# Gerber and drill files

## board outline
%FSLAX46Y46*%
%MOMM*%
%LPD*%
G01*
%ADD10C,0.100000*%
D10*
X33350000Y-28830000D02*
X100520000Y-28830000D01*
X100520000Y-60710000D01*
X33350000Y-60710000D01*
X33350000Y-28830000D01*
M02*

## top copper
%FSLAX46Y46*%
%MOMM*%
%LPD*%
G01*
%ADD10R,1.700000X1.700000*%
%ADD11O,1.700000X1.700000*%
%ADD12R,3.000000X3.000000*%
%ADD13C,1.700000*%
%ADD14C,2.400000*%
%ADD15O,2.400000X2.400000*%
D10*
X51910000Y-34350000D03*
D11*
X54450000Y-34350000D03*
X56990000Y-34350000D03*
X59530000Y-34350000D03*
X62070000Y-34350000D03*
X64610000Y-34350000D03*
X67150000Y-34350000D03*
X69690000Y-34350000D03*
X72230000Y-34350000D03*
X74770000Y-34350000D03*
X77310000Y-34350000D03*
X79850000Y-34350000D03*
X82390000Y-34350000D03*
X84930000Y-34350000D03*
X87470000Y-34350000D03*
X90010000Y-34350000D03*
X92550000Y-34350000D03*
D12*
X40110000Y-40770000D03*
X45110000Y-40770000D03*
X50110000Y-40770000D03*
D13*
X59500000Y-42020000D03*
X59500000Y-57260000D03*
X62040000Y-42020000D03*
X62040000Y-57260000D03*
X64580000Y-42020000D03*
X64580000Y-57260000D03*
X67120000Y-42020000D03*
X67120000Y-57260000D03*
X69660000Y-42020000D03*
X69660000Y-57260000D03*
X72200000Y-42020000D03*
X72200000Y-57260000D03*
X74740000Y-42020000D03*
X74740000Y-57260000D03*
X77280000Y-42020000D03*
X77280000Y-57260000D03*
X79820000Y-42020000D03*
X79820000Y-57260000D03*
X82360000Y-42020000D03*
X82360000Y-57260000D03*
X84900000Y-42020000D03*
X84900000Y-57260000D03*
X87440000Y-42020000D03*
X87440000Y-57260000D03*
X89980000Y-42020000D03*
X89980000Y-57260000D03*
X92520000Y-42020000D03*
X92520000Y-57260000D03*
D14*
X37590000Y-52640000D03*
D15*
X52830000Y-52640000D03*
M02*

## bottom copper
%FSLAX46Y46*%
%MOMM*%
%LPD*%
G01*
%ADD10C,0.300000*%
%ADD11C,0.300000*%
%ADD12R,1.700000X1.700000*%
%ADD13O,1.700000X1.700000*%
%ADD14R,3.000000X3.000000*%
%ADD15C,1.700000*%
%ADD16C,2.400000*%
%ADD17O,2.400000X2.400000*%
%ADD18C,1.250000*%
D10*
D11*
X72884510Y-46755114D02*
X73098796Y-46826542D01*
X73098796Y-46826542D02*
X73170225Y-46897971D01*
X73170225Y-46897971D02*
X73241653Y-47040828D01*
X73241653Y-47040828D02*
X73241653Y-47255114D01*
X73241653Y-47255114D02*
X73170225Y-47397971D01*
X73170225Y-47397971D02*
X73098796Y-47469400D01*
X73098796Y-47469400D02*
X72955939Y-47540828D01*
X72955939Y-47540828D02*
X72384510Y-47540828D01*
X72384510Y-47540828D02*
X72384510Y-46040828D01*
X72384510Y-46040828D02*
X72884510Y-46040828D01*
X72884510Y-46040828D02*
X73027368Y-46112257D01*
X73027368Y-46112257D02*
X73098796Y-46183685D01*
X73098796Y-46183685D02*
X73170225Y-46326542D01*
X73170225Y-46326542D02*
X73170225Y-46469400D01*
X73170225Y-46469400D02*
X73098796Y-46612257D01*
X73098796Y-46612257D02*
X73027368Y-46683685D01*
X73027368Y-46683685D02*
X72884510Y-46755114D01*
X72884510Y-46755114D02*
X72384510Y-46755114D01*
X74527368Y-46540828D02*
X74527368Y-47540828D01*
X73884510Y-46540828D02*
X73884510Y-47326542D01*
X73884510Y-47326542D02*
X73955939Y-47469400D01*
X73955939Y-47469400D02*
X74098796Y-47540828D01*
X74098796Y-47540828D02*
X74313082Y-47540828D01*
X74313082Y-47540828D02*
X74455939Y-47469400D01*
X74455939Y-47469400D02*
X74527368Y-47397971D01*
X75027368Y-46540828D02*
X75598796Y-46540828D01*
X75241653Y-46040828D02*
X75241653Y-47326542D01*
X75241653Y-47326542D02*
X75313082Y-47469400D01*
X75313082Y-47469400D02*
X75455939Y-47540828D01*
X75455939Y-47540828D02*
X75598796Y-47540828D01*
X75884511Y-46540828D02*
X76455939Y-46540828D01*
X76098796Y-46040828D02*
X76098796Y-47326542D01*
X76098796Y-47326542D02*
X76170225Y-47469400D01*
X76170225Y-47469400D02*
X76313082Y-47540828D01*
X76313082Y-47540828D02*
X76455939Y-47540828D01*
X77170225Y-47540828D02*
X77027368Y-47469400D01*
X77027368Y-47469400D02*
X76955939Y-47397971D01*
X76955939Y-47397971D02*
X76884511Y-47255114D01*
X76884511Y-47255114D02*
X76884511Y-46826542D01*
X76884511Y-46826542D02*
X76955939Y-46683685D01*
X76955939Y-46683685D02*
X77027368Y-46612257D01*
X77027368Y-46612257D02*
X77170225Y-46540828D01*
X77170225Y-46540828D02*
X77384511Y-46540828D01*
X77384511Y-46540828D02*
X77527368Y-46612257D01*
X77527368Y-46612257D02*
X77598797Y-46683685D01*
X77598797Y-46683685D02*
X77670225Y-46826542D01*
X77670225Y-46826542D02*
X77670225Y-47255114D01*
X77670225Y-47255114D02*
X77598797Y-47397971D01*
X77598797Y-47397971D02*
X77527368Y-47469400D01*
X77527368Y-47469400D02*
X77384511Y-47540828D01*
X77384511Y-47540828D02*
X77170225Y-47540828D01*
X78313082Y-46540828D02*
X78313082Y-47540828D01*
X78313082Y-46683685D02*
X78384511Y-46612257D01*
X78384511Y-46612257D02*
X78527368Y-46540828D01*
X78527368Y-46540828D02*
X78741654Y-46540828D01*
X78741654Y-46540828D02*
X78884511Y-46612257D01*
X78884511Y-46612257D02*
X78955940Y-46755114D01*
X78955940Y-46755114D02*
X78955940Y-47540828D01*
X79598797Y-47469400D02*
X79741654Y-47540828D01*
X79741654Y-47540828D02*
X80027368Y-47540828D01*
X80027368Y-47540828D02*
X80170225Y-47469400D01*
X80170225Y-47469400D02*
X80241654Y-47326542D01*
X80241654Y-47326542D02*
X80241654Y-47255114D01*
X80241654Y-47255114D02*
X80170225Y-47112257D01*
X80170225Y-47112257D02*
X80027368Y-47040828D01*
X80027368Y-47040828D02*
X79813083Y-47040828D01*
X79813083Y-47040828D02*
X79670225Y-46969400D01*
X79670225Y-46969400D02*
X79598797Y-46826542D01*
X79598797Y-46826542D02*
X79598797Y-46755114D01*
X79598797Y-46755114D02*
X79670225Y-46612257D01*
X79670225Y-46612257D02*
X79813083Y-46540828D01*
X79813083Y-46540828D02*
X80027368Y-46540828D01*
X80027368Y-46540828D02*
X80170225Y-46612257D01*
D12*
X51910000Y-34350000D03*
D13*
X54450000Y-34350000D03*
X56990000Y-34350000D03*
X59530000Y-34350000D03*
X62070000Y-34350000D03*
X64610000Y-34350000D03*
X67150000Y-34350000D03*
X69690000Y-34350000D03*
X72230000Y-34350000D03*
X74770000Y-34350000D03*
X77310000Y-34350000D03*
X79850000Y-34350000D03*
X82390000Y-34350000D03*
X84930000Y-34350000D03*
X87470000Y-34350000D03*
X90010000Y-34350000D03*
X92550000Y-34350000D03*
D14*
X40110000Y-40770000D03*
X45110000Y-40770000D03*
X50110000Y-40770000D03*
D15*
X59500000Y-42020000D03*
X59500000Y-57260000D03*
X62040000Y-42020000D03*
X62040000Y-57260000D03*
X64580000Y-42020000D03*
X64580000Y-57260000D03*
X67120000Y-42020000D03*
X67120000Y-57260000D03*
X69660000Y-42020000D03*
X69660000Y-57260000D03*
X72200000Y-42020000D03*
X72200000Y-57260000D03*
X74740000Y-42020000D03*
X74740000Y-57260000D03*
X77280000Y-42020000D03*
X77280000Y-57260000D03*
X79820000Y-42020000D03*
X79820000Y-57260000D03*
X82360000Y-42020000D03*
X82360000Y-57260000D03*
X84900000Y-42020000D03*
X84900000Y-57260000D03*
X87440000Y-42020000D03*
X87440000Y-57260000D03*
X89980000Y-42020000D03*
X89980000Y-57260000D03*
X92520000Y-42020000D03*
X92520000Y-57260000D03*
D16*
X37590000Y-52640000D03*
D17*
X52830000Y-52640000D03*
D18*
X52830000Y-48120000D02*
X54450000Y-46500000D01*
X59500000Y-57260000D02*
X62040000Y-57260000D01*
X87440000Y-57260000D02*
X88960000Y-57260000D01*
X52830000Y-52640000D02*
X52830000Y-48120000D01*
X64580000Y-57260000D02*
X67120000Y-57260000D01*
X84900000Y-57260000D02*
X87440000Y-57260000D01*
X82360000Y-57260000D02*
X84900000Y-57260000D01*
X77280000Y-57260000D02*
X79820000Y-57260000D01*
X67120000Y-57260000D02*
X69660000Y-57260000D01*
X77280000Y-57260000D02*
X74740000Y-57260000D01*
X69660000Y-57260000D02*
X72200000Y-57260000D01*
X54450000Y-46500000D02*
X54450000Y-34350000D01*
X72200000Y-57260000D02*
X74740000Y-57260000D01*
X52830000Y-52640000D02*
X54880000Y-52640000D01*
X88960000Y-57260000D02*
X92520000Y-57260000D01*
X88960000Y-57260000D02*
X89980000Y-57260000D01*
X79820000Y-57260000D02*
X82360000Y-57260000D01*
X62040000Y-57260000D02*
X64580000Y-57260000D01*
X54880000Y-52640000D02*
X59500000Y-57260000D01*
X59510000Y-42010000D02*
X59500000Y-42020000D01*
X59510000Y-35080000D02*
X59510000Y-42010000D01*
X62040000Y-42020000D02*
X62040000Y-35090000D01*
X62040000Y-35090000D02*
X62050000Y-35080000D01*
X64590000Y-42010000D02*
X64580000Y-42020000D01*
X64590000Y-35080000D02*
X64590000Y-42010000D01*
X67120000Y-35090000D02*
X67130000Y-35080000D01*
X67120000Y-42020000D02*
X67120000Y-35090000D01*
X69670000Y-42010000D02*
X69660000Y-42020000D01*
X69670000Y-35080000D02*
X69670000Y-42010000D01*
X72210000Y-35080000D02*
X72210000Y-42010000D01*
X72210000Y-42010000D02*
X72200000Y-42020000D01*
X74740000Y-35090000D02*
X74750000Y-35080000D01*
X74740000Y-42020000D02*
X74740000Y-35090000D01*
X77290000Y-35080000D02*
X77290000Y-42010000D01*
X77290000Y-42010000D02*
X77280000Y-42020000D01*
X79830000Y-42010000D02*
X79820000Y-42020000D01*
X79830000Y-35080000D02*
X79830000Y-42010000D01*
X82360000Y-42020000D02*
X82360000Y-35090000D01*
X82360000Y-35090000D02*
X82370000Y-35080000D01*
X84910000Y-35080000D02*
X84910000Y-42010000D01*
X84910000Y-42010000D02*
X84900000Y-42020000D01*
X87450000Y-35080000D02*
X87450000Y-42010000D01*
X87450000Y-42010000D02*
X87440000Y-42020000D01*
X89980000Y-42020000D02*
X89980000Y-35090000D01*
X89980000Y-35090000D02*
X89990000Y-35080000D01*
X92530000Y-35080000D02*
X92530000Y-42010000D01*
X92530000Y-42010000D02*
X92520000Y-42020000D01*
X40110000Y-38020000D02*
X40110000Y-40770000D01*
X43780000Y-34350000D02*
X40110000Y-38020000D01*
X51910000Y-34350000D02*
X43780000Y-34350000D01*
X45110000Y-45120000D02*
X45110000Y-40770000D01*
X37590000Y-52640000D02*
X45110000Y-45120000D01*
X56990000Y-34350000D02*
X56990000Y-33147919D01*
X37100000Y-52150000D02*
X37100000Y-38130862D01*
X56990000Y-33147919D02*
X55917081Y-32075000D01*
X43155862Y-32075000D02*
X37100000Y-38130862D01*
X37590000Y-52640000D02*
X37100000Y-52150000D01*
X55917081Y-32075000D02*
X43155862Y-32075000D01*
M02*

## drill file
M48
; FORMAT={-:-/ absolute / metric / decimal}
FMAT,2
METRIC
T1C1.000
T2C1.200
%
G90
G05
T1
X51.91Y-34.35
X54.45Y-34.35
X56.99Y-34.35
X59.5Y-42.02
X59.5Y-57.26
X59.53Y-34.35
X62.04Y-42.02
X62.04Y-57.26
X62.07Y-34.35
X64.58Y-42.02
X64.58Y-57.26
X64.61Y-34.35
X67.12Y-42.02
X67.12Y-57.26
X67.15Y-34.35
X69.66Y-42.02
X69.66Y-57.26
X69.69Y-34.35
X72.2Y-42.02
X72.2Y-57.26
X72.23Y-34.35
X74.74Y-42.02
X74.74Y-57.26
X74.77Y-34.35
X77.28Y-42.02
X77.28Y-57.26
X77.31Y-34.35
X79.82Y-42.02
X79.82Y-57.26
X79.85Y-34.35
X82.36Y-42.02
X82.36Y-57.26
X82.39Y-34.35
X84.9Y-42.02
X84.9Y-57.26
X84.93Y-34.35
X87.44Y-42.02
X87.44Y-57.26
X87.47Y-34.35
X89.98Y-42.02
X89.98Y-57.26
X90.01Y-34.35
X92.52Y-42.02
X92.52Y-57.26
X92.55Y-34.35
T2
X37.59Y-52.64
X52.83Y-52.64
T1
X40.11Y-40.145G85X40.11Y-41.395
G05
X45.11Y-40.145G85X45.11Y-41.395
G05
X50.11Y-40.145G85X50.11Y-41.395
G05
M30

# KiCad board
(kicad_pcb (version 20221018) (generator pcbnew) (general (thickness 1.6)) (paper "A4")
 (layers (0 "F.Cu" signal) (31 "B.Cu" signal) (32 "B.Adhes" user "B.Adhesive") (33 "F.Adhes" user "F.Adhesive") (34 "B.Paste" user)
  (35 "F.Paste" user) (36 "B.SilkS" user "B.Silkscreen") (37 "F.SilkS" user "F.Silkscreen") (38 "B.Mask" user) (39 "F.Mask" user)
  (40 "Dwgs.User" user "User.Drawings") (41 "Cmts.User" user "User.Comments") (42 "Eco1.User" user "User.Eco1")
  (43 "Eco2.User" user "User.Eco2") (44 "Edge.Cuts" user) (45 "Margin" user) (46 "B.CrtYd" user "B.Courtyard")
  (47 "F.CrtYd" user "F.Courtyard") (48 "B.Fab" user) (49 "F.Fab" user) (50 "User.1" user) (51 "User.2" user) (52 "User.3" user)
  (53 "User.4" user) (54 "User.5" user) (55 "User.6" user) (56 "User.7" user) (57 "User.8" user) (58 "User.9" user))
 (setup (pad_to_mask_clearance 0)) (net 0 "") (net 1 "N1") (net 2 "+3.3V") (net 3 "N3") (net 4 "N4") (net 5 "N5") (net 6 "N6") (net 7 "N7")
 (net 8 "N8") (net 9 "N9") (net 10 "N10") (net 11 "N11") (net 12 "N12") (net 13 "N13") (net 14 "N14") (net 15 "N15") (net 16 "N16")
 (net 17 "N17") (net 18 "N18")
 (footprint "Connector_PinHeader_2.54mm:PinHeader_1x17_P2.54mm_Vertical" (layer "F.Cu") (at 51.91 34.35 90)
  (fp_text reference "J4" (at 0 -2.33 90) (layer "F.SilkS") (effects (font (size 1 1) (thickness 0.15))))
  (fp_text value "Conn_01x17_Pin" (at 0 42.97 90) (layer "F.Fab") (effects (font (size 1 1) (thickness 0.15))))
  (pad "1" thru_hole rect (at 0 0 90) (size 1.7 1.7) (drill 1) (layers "*.Cu" "*.Mask") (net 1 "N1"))
  (pad "2" thru_hole oval (at 0 2.54 90) (size 1.7 1.7) (drill 1) (layers "*.Cu" "*.Mask") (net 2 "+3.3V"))
  (pad "3" thru_hole oval (at 0 5.08 90) (size 1.7 1.7) (drill 1) (layers "*.Cu" "*.Mask") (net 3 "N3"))
  (pad "4" thru_hole oval (at 0 7.62 90) (size 1.7 1.7) (drill 1) (layers "*.Cu" "*.Mask") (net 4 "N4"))
  (pad "5" thru_hole oval (at 0 10.16 90) (size 1.7 1.7) (drill 1) (layers "*.Cu" "*.Mask") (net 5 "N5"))
  (pad "6" thru_hole oval (at 0 12.7 90) (size 1.7 1.7) (drill 1) (layers "*.Cu" "*.Mask") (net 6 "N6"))
  (pad "7" thru_hole oval (at 0 15.24 90) (size 1.7 1.7) (drill 1) (layers "*.Cu" "*.Mask") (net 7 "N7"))
  (pad "8" thru_hole oval (at 0 17.78 90) (size 1.7 1.7) (drill 1) (layers "*.Cu" "*.Mask") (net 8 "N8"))
  (pad "9" thru_hole oval (at 0 20.32 90) (size 1.7 1.7) (drill 1) (layers "*.Cu" "*.Mask") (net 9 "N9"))
  (pad "10" thru_hole oval (at 0 22.86 90) (size 1.7 1.7) (drill 1) (layers "*.Cu" "*.Mask") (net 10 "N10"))
  (pad "11" thru_hole oval (at 0 25.4 90) (size 1.7 1.7) (drill 1) (layers "*.Cu" "*.Mask") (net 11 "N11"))
  (pad "12" thru_hole oval (at 0 27.94 90) (size 1.7 1.7) (drill 1) (layers "*.Cu" "*.Mask") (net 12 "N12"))
  (pad "13" thru_hole oval (at 0 30.48 90) (size 1.7 1.7) (drill 1) (layers "*.Cu" "*.Mask") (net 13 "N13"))
  (pad "14" thru_hole oval (at 0 33.02 90) (size 1.7 1.7) (drill 1) (layers "*.Cu" "*.Mask") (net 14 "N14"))
  (pad "15" thru_hole oval (at 0 35.56 90) (size 1.7 1.7) (drill 1) (layers "*.Cu" "*.Mask") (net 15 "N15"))
  (pad "16" thru_hole oval (at 0 38.1 90) (size 1.7 1.7) (drill 1) (layers "*.Cu" "*.Mask") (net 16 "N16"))
  (pad "17" thru_hole oval (at 0 40.64 90) (size 1.7 1.7) (drill 1) (layers "*.Cu" "*.Mask") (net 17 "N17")))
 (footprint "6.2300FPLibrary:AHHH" (layer "F.Cu") (at 40.11 40.77)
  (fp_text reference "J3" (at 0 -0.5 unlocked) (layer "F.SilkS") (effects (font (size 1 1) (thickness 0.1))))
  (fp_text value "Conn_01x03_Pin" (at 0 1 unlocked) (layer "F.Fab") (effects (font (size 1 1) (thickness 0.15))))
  (pad "1" thru_hole rect (at 0 0) (size 3 3) (drill oval 1 2.25) (layers "*.Cu" "*.Mask") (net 1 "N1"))
  (pad "2" thru_hole rect (at 5 0) (size 3 3) (drill oval 1 2.25) (layers "*.Cu" "*.Mask") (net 3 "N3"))
  (pad "3" thru_hole rect (at 10 0) (size 3 3) (drill oval 1 2.25) (layers "*.Cu" "*.Mask") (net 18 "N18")))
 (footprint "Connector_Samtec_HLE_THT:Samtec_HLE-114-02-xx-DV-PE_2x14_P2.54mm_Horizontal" (layer "F.Cu") (at 59.5 42.02)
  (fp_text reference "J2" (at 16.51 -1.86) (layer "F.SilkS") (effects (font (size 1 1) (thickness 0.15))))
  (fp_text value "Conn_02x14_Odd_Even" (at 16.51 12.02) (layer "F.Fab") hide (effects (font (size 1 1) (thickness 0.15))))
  (pad "1" thru_hole circle (at 0 0) (size 1.7 1.7) (drill 1) (layers "*.Cu" "*.Mask") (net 4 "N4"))
  (pad "2" thru_hole circle (at 0 15.24) (size 1.7 1.7) (drill 1) (layers "*.Cu" "*.Mask") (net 2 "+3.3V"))
  (pad "3" thru_hole circle (at 2.54 0) (size 1.7 1.7) (drill 1) (layers "*.Cu" "*.Mask") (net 5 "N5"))
  (pad "4" thru_hole circle (at 2.54 15.24) (size 1.7 1.7) (drill 1) (layers "*.Cu" "*.Mask") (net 2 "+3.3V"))
  (pad "5" thru_hole circle (at 5.08 0) (size 1.7 1.7) (drill 1) (layers "*.Cu" "*.Mask") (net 6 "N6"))
  (pad "6" thru_hole circle (at 5.08 15.24) (size 1.7 1.7) (drill 1) (layers "*.Cu" "*.Mask") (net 2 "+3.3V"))
  (pad "7" thru_hole circle (at 7.62 0) (size 1.7 1.7) (drill 1) (layers "*.Cu" "*.Mask") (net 7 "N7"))
  (pad "8" thru_hole circle (at 7.62 15.24) (size 1.7 1.7) (drill 1) (layers "*.Cu" "*.Mask") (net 2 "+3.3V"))
  (pad "9" thru_hole circle (at 10.16 0) (size 1.7 1.7) (drill 1) (layers "*.Cu" "*.Mask") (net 8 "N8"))
  (pad "10" thru_hole circle (at 10.16 15.24) (size 1.7 1.7) (drill 1) (layers "*.Cu" "*.Mask") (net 2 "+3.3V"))
  (pad "11" thru_hole circle (at 12.7 0) (size 1.7 1.7) (drill 1) (layers "*.Cu" "*.Mask") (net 9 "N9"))
  (pad "12" thru_hole circle (at 12.7 15.24) (size 1.7 1.7) (drill 1) (layers "*.Cu" "*.Mask") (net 2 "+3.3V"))
  (pad "13" thru_hole circle (at 15.24 0) (size 1.7 1.7) (drill 1) (layers "*.Cu" "*.Mask") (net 10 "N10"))
  (pad "14" thru_hole circle (at 15.24 15.24) (size 1.7 1.7) (drill 1) (layers "*.Cu" "*.Mask") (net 2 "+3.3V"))
  (pad "15" thru_hole circle (at 17.78 0) (size 1.7 1.7) (drill 1) (layers "*.Cu" "*.Mask") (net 11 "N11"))
  (pad "16" thru_hole circle (at 17.78 15.24) (size 1.7 1.7) (drill 1) (layers "*.Cu" "*.Mask") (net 2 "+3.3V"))
  (pad "17" thru_hole circle (at 20.32 0) (size 1.7 1.7) (drill 1) (layers "*.Cu" "*.Mask") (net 12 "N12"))
  (pad "18" thru_hole circle (at 20.32 15.24) (size 1.7 1.7) (drill 1) (layers "*.Cu" "*.Mask") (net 2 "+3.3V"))
  (pad "19" thru_hole circle (at 22.86 0) (size 1.7 1.7) (drill 1) (layers "*.Cu" "*.Mask") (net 13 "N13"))
  (pad "20" thru_hole circle (at 22.86 15.24) (size 1.7 1.7) (drill 1) (layers "*.Cu" "*.Mask") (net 2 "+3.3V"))
  (pad "21" thru_hole circle (at 25.4 0) (size 1.7 1.7) (drill 1) (layers "*.Cu" "*.Mask") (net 14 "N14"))
  (pad "22" thru_hole circle (at 25.4 15.24) (size 1.7 1.7) (drill 1) (layers "*.Cu" "*.Mask") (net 2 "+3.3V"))
  (pad "23" thru_hole circle (at 27.94 0) (size 1.7 1.7) (drill 1) (layers "*.Cu" "*.Mask") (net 15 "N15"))
  (pad "24" thru_hole circle (at 27.94 15.24) (size 1.7 1.7) (drill 1) (layers "*.Cu" "*.Mask") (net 2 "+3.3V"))
  (pad "25" thru_hole circle (at 30.48 0) (size 1.7 1.7) (drill 1) (layers "*.Cu" "*.Mask") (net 16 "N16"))
  (pad "26" thru_hole circle (at 30.48 15.24) (size 1.7 1.7) (drill 1) (layers "*.Cu" "*.Mask") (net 2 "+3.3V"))
  (pad "27" thru_hole circle (at 33.02 0) (size 1.7 1.7) (drill 1) (layers "*.Cu" "*.Mask") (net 17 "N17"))
  (pad "28" thru_hole circle (at 33.02 15.24) (size 1.7 1.7) (drill 1) (layers "*.Cu" "*.Mask") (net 2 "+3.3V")))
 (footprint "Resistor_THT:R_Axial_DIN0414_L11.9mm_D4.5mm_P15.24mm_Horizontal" (layer "F.Cu") (at 37.59 52.64)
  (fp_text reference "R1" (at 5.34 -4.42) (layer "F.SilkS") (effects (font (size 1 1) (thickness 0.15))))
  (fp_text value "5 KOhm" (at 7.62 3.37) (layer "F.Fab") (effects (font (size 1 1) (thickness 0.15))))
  (pad "1" thru_hole circle (at 0 0) (size 2.4 2.4) (drill 1.2) (layers "*.Cu" "*.Mask") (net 3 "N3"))
  (pad "2" thru_hole oval (at 15.24 0) (size 2.4 2.4) (drill 1.2) (layers "*.Cu" "*.Mask") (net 2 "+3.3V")))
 (gr_rect (start 33.35 28.83) (end 100.52 60.71) (stroke (width 0.1) (type default)) (fill none) (layer "Edge.Cuts"))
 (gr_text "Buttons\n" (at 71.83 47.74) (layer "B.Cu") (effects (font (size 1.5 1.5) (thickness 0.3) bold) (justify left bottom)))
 (segment (start 52.83 48.12) (end 54.45 46.5) (width 1.25) (layer "B.Cu") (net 2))
 (segment (start 59.5 57.26) (end 62.04 57.26) (width 1.25) (layer "B.Cu") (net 2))
 (segment (start 87.44 57.26) (end 88.96 57.26) (width 1.25) (layer "B.Cu") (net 2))
 (segment (start 52.83 52.64) (end 52.83 48.12) (width 1.25) (layer "B.Cu") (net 2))
 (segment (start 64.58 57.26) (end 67.12 57.26) (width 1.25) (layer "B.Cu") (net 2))
 (segment (start 84.9 57.26) (end 87.44 57.26) (width 1.25) (layer "B.Cu") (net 2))
 (segment (start 82.36 57.26) (end 84.9 57.26) (width 1.25) (layer "B.Cu") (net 2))
 (segment (start 77.28 57.26) (end 79.82 57.26) (width 1.25) (layer "B.Cu") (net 2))
 (segment (start 67.12 57.26) (end 69.66 57.26) (width 1.25) (layer "B.Cu") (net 2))
 (segment (start 77.28 57.26) (end 74.74 57.26) (width 1.25) (layer "B.Cu") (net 2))
 (segment (start 69.66 57.26) (end 72.2 57.26) (width 1.25) (layer "B.Cu") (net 2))
 (segment (start 54.45 46.5) (end 54.45 34.35) (width 1.25) (layer "B.Cu") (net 2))
 (segment (start 72.2 57.26) (end 74.74 57.26) (width 1.25) (layer "B.Cu") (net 2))
 (segment (start 52.83 52.64) (end 54.88 52.64) (width 1.25) (layer "B.Cu") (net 2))
 (segment (start 88.96 57.26) (end 92.52 57.26) (width 1.25) (layer "B.Cu") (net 2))
 (segment (start 88.96 57.26) (end 89.98 57.26) (width 1.25) (layer "B.Cu") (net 2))
 (segment (start 79.82 57.26) (end 82.36 57.26) (width 1.25) (layer "B.Cu") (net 2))
 (segment (start 62.04 57.26) (end 64.58 57.26) (width 1.25) (layer "B.Cu") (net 2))
 (segment (start 54.88 52.64) (end 59.5 57.26) (width 1.25) (layer "B.Cu") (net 2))
 (segment (start 59.51 42.01) (end 59.5 42.02) (width 1.25) (layer "B.Cu") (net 4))
 (segment (start 59.51 35.08) (end 59.51 42.01) (width 1.25) (layer "B.Cu") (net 4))
 (segment (start 62.04 42.02) (end 62.04 35.09) (width 1.25) (layer "B.Cu") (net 5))
 (segment (start 62.04 35.09) (end 62.05 35.08) (width 1.25) (layer "B.Cu") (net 5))
 (segment (start 64.59 42.01) (end 64.58 42.02) (width 1.25) (layer "B.Cu") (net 6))
 (segment (start 64.59 35.08) (end 64.59 42.01) (width 1.25) (layer "B.Cu") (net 6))
 (segment (start 67.12 35.09) (end 67.13 35.08) (width 1.25) (layer "B.Cu") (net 7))
 (segment (start 67.12 42.02) (end 67.12 35.09) (width 1.25) (layer "B.Cu") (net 7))
 (segment (start 69.67 42.01) (end 69.66 42.02) (width 1.25) (layer "B.Cu") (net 8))
 (segment (start 69.67 35.08) (end 69.67 42.01) (width 1.25) (layer "B.Cu") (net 8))
 (segment (start 72.21 35.08) (end 72.21 42.01) (width 1.25) (layer "B.Cu") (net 9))
 (segment (start 72.21 42.01) (end 72.2 42.02) (width 1.25) (layer "B.Cu") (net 9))
 (segment (start 74.74 35.09) (end 74.75 35.08) (width 1.25) (layer "B.Cu") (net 10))
 (segment (start 74.74 42.02) (end 74.74 35.09) (width 1.25) (layer "B.Cu") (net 10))
 (segment (start 77.29 35.08) (end 77.29 42.01) (width 1.25) (layer "B.Cu") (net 11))
 (segment (start 77.29 42.01) (end 77.28 42.02) (width 1.25) (layer "B.Cu") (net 11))
 (segment (start 79.83 42.01) (end 79.82 42.02) (width 1.25) (layer "B.Cu") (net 12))
 (segment (start 79.83 35.08) (end 79.83 42.01) (width 1.25) (layer "B.Cu") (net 12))
 (segment (start 82.36 42.02) (end 82.36 35.09) (width 1.25) (layer "B.Cu") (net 13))
 (segment (start 82.36 35.09) (end 82.37 35.08) (width 1.25) (layer "B.Cu") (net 13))
 (segment (start 84.91 35.08) (end 84.91 42.01) (width 1.25) (layer "B.Cu") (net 14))
 (segment (start 84.91 42.01) (end 84.9 42.02) (width 1.25) (layer "B.Cu") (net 14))
 (segment (start 87.45 35.08) (end 87.45 42.01) (width 1.25) (layer "B.Cu") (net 15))
 (segment (start 87.45 42.01) (end 87.44 42.02) (width 1.25) (layer "B.Cu") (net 15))
 (segment (start 89.98 42.02) (end 89.98 35.09) (width 1.25) (layer "B.Cu") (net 16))
 (segment (start 89.98 35.09) (end 89.99 35.08) (width 1.25) (layer "B.Cu") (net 16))
 (segment (start 92.53 35.08) (end 92.53 42.01) (width 1.25) (layer "B.Cu") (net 17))
 (segment (start 92.53 42.01) (end 92.52 42.02) (width 1.25) (layer "B.Cu") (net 17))
 (segment (start 40.11 38.02) (end 40.11 40.77) (width 1.25) (layer "B.Cu") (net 1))
 (segment (start 43.78 34.35) (end 40.11 38.02) (width 1.25) (layer "B.Cu") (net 1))
 (segment (start 51.91 34.35) (end 43.78 34.35) (width 1.25) (layer "B.Cu") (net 1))
 (segment (start 45.11 45.12) (end 45.11 40.77) (width 1.25) (layer "B.Cu") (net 3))
 (segment (start 37.59 52.64) (end 45.11 45.12) (width 1.25) (layer "B.Cu") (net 3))
 (segment (start 56.99 34.35) (end 56.99 33.147919) (width 1.25) (layer "B.Cu") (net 3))
 (segment (start 37.1 52.15) (end 37.1 38.130862) (width 1.25) (layer "B.Cu") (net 3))
 (segment (start 56.99 33.147919) (end 55.917081 32.075) (width 1.25) (layer "B.Cu") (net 3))
 (segment (start 43.155862 32.075) (end 37.1 38.130862) (width 1.25) (layer "B.Cu") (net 3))
 (segment (start 37.59 52.64) (end 37.1 52.15) (width 1.25) (layer "B.Cu") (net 3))
 (segment (start 55.917081 32.075) (end 43.155862 32.075) (width 1.25) (layer "B.Cu") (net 3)))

